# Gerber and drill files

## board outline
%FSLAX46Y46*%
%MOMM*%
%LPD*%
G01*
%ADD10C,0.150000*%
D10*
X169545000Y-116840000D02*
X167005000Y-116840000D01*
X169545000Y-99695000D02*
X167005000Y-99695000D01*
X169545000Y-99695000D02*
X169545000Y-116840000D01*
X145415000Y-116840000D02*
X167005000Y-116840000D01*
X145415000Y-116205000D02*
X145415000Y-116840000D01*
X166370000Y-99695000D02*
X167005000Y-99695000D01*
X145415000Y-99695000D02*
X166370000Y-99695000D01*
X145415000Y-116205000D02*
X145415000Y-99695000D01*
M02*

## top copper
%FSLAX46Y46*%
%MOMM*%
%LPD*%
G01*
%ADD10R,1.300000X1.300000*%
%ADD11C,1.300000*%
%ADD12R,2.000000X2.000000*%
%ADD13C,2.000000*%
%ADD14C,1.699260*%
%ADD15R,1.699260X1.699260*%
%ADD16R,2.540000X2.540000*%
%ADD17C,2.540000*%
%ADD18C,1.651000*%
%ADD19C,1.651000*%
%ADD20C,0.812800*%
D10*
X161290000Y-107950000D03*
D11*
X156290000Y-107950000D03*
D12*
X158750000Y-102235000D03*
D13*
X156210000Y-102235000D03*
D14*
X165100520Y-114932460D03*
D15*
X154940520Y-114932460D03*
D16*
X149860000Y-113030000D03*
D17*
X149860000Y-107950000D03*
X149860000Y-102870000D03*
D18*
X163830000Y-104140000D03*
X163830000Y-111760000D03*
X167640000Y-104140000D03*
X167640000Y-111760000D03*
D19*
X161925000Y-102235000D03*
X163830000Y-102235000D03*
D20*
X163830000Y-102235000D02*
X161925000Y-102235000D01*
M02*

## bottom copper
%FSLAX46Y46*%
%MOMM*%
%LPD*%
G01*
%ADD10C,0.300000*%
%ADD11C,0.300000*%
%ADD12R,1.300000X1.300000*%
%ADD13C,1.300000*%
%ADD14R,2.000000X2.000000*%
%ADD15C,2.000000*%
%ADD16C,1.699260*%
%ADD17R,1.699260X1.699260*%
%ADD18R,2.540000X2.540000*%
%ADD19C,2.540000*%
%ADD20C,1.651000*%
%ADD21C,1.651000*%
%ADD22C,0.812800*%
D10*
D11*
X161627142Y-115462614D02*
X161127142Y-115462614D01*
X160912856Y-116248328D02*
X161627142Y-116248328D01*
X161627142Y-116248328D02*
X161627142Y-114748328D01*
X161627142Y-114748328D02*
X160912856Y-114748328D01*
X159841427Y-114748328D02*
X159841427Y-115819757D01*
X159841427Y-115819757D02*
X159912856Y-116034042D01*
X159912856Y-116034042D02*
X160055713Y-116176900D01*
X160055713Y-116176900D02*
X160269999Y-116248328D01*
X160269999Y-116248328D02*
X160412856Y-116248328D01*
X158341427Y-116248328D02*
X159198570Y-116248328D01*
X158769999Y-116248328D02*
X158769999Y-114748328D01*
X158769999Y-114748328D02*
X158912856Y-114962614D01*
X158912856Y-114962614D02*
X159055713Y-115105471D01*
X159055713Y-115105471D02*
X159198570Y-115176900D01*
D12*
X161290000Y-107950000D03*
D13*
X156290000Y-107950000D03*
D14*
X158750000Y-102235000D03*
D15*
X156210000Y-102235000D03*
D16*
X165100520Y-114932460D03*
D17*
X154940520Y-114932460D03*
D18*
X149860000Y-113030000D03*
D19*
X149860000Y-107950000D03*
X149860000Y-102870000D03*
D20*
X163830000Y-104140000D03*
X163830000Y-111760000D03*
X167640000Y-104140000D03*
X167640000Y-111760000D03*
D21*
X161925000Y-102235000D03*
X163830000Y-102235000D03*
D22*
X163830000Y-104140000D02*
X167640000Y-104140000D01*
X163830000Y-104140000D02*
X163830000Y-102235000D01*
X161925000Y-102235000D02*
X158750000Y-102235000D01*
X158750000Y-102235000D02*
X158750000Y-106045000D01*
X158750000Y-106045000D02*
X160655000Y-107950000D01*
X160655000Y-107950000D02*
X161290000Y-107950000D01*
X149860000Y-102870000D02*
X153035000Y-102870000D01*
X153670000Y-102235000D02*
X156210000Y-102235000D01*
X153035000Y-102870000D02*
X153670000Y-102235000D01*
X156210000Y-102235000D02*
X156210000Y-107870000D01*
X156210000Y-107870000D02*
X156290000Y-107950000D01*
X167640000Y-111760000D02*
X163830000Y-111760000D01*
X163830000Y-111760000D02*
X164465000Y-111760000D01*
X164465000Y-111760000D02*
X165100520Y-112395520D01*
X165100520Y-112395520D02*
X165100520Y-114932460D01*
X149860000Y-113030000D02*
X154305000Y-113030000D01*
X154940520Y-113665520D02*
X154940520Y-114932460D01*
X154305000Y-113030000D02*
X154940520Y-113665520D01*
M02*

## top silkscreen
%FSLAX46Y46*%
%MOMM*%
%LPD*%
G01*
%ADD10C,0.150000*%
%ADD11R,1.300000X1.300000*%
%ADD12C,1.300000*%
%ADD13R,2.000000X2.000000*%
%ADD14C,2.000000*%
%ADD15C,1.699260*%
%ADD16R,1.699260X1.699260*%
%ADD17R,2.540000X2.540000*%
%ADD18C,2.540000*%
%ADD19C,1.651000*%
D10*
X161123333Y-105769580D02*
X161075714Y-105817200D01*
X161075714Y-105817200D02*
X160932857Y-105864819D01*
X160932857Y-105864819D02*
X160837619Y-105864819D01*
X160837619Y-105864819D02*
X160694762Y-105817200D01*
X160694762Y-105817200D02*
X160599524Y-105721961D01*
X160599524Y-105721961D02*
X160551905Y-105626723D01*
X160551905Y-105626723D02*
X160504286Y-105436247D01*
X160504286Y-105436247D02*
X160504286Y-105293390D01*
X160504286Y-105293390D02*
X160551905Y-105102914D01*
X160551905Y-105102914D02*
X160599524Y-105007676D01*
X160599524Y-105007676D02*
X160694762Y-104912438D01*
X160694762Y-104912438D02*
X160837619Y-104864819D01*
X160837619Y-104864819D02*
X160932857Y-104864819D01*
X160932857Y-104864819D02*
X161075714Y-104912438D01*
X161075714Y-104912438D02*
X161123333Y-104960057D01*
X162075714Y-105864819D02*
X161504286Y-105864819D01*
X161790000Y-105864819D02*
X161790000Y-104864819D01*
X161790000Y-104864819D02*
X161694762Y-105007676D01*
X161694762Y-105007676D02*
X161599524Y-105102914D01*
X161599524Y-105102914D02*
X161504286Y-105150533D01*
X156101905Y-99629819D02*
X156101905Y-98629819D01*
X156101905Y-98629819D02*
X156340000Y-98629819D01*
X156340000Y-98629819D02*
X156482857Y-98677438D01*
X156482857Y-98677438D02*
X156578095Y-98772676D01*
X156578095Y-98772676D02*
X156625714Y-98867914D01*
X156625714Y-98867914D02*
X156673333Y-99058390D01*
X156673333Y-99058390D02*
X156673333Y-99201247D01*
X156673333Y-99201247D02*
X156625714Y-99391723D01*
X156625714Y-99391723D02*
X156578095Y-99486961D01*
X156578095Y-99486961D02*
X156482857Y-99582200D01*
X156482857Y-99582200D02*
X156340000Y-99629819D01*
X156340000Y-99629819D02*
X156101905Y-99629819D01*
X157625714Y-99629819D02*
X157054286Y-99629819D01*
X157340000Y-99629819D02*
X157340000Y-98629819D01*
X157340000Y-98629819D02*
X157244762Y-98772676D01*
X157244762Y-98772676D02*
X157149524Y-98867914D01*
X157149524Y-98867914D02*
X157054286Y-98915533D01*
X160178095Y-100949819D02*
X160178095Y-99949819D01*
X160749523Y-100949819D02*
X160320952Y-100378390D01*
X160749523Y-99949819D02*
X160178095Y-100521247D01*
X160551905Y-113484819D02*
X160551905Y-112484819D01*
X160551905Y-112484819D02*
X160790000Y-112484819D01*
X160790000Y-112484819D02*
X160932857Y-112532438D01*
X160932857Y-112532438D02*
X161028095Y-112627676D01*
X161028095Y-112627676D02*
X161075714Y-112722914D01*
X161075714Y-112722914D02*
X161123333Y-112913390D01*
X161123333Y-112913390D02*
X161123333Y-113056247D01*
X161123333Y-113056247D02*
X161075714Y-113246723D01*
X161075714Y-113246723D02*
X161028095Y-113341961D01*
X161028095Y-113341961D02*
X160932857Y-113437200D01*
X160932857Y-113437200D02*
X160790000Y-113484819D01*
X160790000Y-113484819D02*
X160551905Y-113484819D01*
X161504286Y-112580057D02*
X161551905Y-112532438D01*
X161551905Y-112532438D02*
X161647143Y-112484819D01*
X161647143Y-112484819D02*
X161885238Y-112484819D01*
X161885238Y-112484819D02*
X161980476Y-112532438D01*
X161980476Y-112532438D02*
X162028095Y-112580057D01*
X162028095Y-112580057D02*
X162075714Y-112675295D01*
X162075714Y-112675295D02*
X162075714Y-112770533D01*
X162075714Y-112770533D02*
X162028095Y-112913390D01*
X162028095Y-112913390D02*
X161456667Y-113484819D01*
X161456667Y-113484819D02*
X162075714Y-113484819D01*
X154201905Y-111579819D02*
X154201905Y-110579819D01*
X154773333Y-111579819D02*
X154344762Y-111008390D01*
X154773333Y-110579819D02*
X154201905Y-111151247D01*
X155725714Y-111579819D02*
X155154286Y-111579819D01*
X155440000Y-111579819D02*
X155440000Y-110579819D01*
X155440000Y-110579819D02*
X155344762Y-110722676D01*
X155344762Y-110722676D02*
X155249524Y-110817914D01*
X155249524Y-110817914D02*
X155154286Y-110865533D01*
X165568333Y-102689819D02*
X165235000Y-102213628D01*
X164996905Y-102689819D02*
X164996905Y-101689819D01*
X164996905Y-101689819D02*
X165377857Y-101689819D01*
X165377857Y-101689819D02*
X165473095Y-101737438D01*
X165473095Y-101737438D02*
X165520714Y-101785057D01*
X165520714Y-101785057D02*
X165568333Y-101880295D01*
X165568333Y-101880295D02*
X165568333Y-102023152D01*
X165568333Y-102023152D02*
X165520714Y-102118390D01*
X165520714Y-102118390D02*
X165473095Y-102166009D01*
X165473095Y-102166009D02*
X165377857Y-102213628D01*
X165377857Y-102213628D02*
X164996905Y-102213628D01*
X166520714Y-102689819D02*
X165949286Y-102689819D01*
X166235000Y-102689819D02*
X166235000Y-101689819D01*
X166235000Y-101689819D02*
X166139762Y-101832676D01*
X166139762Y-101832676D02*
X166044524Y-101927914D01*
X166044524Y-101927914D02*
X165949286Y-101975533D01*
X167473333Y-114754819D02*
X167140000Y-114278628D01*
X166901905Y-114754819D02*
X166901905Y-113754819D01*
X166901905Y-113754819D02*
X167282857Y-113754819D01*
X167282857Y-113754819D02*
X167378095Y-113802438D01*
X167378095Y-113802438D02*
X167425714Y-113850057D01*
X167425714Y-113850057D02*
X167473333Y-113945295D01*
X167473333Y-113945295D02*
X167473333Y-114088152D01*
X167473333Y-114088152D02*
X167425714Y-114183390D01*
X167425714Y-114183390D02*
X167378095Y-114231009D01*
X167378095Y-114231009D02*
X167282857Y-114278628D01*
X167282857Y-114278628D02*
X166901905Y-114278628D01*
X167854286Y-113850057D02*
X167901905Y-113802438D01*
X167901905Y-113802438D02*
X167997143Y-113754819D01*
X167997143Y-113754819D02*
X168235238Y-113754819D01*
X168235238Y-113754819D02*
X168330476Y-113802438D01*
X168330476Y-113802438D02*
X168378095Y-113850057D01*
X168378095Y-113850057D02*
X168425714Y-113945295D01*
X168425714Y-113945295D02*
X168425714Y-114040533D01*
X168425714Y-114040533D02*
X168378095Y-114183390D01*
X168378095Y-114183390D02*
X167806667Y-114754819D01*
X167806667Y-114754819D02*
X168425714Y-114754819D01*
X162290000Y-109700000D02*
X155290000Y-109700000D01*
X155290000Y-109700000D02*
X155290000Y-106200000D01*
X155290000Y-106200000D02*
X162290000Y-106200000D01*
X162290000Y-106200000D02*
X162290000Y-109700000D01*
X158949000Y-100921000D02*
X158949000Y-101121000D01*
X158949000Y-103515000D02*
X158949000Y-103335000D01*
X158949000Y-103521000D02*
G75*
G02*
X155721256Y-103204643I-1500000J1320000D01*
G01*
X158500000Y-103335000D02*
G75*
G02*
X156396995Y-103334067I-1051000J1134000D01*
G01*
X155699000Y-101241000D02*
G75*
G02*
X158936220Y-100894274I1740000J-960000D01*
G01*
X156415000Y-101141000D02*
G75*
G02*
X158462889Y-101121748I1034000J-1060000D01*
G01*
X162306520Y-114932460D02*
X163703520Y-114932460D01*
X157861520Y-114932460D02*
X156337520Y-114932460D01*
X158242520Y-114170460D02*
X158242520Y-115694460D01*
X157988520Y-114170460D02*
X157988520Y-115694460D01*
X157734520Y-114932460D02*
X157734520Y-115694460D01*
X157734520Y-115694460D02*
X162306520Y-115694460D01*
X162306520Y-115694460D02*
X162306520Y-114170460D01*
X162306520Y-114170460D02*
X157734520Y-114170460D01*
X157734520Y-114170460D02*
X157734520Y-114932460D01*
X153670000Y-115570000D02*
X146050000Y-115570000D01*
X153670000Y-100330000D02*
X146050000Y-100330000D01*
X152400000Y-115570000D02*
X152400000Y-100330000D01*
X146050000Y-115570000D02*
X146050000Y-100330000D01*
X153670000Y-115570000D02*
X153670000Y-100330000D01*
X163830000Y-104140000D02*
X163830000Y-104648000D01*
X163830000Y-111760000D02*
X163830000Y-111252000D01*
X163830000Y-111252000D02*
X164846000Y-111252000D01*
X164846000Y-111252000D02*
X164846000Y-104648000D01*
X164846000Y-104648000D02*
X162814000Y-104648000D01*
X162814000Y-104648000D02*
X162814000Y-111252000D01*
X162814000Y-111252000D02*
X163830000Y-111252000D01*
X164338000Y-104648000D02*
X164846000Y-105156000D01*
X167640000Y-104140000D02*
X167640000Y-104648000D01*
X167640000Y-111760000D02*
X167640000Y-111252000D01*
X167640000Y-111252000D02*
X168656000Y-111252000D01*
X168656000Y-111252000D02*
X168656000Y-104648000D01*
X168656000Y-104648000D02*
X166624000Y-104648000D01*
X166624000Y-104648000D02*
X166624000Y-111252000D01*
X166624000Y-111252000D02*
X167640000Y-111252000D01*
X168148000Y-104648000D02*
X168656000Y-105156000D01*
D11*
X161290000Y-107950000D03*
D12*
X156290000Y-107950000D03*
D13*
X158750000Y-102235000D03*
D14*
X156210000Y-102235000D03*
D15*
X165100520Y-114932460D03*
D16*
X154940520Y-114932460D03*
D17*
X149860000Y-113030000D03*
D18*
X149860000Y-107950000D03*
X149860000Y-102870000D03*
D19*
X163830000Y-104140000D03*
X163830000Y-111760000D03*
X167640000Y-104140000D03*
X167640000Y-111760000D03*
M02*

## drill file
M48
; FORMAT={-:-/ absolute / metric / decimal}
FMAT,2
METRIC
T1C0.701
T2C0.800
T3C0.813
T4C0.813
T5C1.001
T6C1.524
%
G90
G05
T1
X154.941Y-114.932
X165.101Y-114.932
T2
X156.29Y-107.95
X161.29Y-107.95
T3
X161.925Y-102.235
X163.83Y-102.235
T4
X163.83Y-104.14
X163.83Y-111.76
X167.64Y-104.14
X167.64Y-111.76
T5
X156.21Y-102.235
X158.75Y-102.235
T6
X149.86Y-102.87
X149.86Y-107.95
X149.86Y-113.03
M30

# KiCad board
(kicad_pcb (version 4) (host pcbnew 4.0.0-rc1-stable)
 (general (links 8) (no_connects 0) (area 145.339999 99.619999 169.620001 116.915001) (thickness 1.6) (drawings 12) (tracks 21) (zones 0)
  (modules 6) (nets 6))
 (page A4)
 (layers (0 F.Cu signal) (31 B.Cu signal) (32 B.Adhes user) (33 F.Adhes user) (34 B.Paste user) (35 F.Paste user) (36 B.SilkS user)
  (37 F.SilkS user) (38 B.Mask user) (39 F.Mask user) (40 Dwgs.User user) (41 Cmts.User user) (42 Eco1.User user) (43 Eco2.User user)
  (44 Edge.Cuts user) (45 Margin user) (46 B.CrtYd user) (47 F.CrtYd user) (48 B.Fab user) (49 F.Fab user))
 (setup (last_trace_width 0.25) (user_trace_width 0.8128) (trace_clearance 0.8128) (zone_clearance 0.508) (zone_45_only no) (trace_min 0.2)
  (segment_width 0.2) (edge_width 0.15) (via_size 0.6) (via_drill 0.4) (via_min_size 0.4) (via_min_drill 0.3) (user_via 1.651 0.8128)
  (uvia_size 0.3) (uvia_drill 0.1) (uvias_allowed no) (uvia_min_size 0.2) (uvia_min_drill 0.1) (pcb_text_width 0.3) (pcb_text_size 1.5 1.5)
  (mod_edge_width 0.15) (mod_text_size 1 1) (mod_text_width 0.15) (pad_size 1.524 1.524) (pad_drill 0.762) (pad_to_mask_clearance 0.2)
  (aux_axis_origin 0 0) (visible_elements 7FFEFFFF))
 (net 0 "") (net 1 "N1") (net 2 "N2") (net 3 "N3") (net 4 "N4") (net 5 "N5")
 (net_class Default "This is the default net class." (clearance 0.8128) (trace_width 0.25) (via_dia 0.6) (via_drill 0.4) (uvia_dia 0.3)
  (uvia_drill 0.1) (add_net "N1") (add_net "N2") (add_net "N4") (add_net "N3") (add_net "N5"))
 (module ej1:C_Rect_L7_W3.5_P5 (layer F.Cu) (at 161.29 107.95 180)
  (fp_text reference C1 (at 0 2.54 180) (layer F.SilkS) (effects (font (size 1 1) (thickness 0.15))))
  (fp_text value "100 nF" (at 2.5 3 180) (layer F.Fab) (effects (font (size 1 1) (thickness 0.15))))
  (fp_line (start -1 -1.75) (end 6 -1.75) (layer F.SilkS) (width 0.15))
  (fp_line (start 6 -1.75) (end 6 1.75) (layer F.SilkS) (width 0.15))
  (fp_line (start 6 1.75) (end -1 1.75) (layer F.SilkS) (width 0.15))
  (fp_line (start -1 1.75) (end -1 -1.75) (layer F.SilkS) (width 0.15))
  (pad 1 thru_hole rect (at 0 0 180) (size 1.3 1.3) (drill 0.8) (layers *.Cu *.Mask F.SilkS) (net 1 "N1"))
  (pad 2 thru_hole circle (at 5 0 180) (size 1.3 1.3) (drill 0.8) (layers *.Cu *.Mask F.SilkS) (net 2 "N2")))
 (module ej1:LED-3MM (layer F.Cu) (at 158.75 102.235 180)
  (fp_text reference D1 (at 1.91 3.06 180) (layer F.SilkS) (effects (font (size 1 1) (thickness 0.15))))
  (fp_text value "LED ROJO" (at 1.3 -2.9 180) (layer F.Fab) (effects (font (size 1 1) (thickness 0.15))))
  (fp_line (start -0.199 1.314) (end -0.199 1.114) (layer F.SilkS) (width 0.15))
  (fp_line (start -0.199 -1.28) (end -0.199 -1.1) (layer F.SilkS) (width 0.15))
  (fp_arc (start 1.301 0.034) (end -0.199 -1.286) (angle 108.5) (layer F.SilkS) (width 0.15))
  (fp_arc (start 1.301 0.034) (end 0.25 -1.1) (angle 85.7) (layer F.SilkS) (width 0.15))
  (fp_arc (start 1.311 0.034) (end 3.051 0.994) (angle 110) (layer F.SilkS) (width 0.15))
  (fp_arc (start 1.301 0.034) (end 2.335 1.094) (angle 87.5) (layer F.SilkS) (width 0.15))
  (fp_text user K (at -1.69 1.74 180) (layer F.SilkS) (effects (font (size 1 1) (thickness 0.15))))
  (pad 1 thru_hole rect (at 0 0 270) (size 2 2) (drill 1.00076) (layers *.Cu *.Mask F.SilkS) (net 1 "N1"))
  (pad 2 thru_hole circle (at 2.54 0 180) (size 2 2) (drill 1.00076) (layers *.Cu *.Mask F.SilkS) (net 2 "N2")))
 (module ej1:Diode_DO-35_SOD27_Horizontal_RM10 (layer F.Cu) (at 154.94 114.935)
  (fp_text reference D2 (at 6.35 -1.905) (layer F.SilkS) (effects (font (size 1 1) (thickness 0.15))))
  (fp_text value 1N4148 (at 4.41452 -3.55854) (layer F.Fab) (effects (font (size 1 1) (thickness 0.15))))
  (fp_line (start 7.36652 -0.00254) (end 8.76352 -0.00254) (layer F.SilkS) (width 0.15))
  (fp_line (start 2.92152 -0.00254) (end 1.39752 -0.00254) (layer F.SilkS) (width 0.15))
  (fp_line (start 3.30252 -0.76454) (end 3.30252 0.75946) (layer F.SilkS) (width 0.15))
  (fp_line (start 3.04852 -0.76454) (end 3.04852 0.75946) (layer F.SilkS) (width 0.15))
  (fp_line (start 2.79452 -0.00254) (end 2.79452 0.75946) (layer F.SilkS) (width 0.15))
  (fp_line (start 2.79452 0.75946) (end 7.36652 0.75946) (layer F.SilkS) (width 0.15))
  (fp_line (start 7.36652 0.75946) (end 7.36652 -0.76454) (layer F.SilkS) (width 0.15))
  (fp_line (start 7.36652 -0.76454) (end 2.79452 -0.76454) (layer F.SilkS) (width 0.15))
  (fp_line (start 2.79452 -0.76454) (end 2.79452 -0.00254) (layer F.SilkS) (width 0.15))
  (pad 2 thru_hole circle (at 10.16052 -0.00254 180) (size 1.69926 1.69926) (drill 0.70104) (layers *.Cu *.Mask F.SilkS) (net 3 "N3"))
  (pad 1 thru_hole rect (at 0.00052 -0.00254 180) (size 1.69926 1.69926) (drill 0.70104) (layers *.Cu *.Mask F.SilkS) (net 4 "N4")))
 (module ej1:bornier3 (layer F.Cu) (at 149.86 107.95 90)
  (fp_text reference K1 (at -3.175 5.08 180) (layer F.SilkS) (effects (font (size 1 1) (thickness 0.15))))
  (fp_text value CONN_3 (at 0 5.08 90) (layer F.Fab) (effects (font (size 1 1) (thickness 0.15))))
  (fp_line (start -7.62 3.81) (end -7.62 -3.81) (layer F.SilkS) (width 0.15))
  (fp_line (start 7.62 3.81) (end 7.62 -3.81) (layer F.SilkS) (width 0.15))
  (fp_line (start -7.62 2.54) (end 7.62 2.54) (layer F.SilkS) (width 0.15))
  (fp_line (start -7.62 -3.81) (end 7.62 -3.81) (layer F.SilkS) (width 0.15))
  (fp_line (start -7.62 3.81) (end 7.62 3.81) (layer F.SilkS) (width 0.15))
  (pad 1 thru_hole rect (at -5.08 0 90) (size 2.54 2.54) (drill 1.524) (layers *.Cu *.Mask F.SilkS) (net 4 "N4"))
  (pad 2 thru_hole circle (at 0 0 90) (size 2.54 2.54) (drill 1.524) (layers *.Cu *.Mask F.SilkS) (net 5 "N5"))
  (pad 3 thru_hole circle (at 5.08 0 90) (size 2.54 2.54) (drill 1.524) (layers *.Cu *.Mask F.SilkS) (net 2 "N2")))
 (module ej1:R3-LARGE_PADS (layer F.Cu) (at 163.83 107.95 270)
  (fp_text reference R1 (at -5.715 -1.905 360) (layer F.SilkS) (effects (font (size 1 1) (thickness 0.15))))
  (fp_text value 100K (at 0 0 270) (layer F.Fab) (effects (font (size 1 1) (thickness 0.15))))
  (fp_line (start -3.81 0) (end -3.302 0) (layer F.SilkS) (width 0.15))
  (fp_line (start 3.81 0) (end 3.302 0) (layer F.SilkS) (width 0.15))
  (fp_line (start 3.302 0) (end 3.302 -1.016) (layer F.SilkS) (width 0.15))
  (fp_line (start 3.302 -1.016) (end -3.302 -1.016) (layer F.SilkS) (width 0.15))
  (fp_line (start -3.302 -1.016) (end -3.302 1.016) (layer F.SilkS) (width 0.15))
  (fp_line (start -3.302 1.016) (end 3.302 1.016) (layer F.SilkS) (width 0.15))
  (fp_line (start 3.302 1.016) (end 3.302 0) (layer F.SilkS) (width 0.15))
  (fp_line (start -3.302 -0.508) (end -2.794 -1.016) (layer F.SilkS) (width 0.15))
  (pad 1 thru_hole circle (at -3.81 0 270) (size 1.651 1.651) (drill 0.8128) (layers *.Cu *.Mask F.SilkS) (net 1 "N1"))
  (pad 2 thru_hole circle (at 3.81 0 270) (size 1.651 1.651) (drill 0.8128) (layers *.Cu *.Mask F.SilkS) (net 3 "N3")))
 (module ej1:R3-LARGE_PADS (layer F.Cu) (at 167.64 107.95 270)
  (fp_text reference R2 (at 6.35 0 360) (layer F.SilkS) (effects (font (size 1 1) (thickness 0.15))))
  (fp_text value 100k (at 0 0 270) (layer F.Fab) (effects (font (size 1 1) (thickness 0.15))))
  (fp_line (start -3.81 0) (end -3.302 0) (layer F.SilkS) (width 0.15))
  (fp_line (start 3.81 0) (end 3.302 0) (layer F.SilkS) (width 0.15))
  (fp_line (start 3.302 0) (end 3.302 -1.016) (layer F.SilkS) (width 0.15))
  (fp_line (start 3.302 -1.016) (end -3.302 -1.016) (layer F.SilkS) (width 0.15))
  (fp_line (start -3.302 -1.016) (end -3.302 1.016) (layer F.SilkS) (width 0.15))
  (fp_line (start -3.302 1.016) (end 3.302 1.016) (layer F.SilkS) (width 0.15))
  (fp_line (start 3.302 1.016) (end 3.302 0) (layer F.SilkS) (width 0.15))
  (fp_line (start -3.302 -0.508) (end -2.794 -1.016) (layer F.SilkS) (width 0.15))
  (pad 1 thru_hole circle (at -3.81 0 270) (size 1.651 1.651) (drill 0.8128) (layers *.Cu *.Mask F.SilkS) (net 1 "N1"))
  (pad 2 thru_hole circle (at 3.81 0 270) (size 1.651 1.651) (drill 0.8128) (layers *.Cu *.Mask F.SilkS) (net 3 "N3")))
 (gr_line (start 169.545 116.84) (end 167.005 116.84) (angle 90) (layer Edge.Cuts) (width 0.15))
 (gr_line (start 169.545 99.695) (end 167.005 99.695) (angle 90) (layer Edge.Cuts) (width 0.15))
 (gr_line (start 169.545 99.695) (end 169.545 116.84) (angle 90) (layer Edge.Cuts) (width 0.15))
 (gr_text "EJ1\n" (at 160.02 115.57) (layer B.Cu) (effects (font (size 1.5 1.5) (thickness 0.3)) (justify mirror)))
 (gr_line (start 145.415 116.84) (end 167.005 116.84) (angle 90) (layer Edge.Cuts) (width 0.15))
 (gr_line (start 145.415 116.205) (end 145.415 116.84) (angle 90) (layer Edge.Cuts) (width 0.15))
 (gr_line (start 166.37 99.695) (end 167.005 99.695) (angle 90) (layer Edge.Cuts) (width 0.15))
 (gr_line (start 145.415 99.695) (end 166.37 99.695) (angle 90) (layer Edge.Cuts) (width 0.15))
 (gr_line (start 145.415 116.205) (end 145.415 99.695) (angle 90) (layer Edge.Cuts) (width 0.15))
 (segment (start 163.83 104.14) (end 167.64 104.14) (width 0.8128) (layer B.Cu) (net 1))
 (segment (start 163.83 104.14) (end 163.83 102.235) (width 0.8128) (layer B.Cu) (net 1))
 (segment (start 161.925 102.235) (end 158.75 102.235) (width 0.8128) (layer B.Cu) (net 1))
 (via (at 161.925 102.235) (size 1.651) (drill 0.8128) (layers F.Cu B.Cu) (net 1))
 (segment (start 163.83 102.235) (end 161.925 102.235) (width 0.8128) (layer F.Cu) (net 1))
 (via (at 163.83 102.235) (size 1.651) (drill 0.8128) (layers F.Cu B.Cu) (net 1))
 (segment (start 158.75 102.235) (end 158.75 106.045) (width 0.8128) (layer B.Cu) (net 1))
 (segment (start 158.75 106.045) (end 160.655 107.95) (width 0.8128) (layer B.Cu) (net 1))
 (segment (start 160.655 107.95) (end 161.29 107.95) (width 0.8128) (layer B.Cu) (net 1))
 (segment (start 149.86 102.87) (end 153.035 102.87) (width 0.8128) (layer B.Cu) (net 2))
 (segment (start 153.67 102.235) (end 156.21 102.235) (width 0.8128) (layer B.Cu) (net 2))
 (segment (start 153.035 102.87) (end 153.67 102.235) (width 0.8128) (layer B.Cu) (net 2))
 (segment (start 156.21 102.235) (end 156.21 107.87) (width 0.8128) (layer B.Cu) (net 2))
 (segment (start 156.21 107.87) (end 156.29 107.95) (width 0.8128) (layer B.Cu) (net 2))
 (segment (start 167.64 111.76) (end 163.83 111.76) (width 0.8128) (layer B.Cu) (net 3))
 (segment (start 163.83 111.76) (end 164.465 111.76) (width 0.8128) (layer B.Cu) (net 3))
 (segment (start 164.465 111.76) (end 165.10052 112.39552) (width 0.8128) (layer B.Cu) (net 3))
 (segment (start 165.10052 112.39552) (end 165.10052 114.93246) (width 0.8128) (layer B.Cu) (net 3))
 (segment (start 149.86 113.03) (end 154.305 113.03) (width 0.8128) (layer B.Cu) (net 4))
 (segment (start 154.94052 113.66552) (end 154.94052 114.93246) (width 0.8128) (layer B.Cu) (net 4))
 (segment (start 154.305 113.03) (end 154.94052 113.66552) (width 0.8128) (layer B.Cu) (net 4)))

